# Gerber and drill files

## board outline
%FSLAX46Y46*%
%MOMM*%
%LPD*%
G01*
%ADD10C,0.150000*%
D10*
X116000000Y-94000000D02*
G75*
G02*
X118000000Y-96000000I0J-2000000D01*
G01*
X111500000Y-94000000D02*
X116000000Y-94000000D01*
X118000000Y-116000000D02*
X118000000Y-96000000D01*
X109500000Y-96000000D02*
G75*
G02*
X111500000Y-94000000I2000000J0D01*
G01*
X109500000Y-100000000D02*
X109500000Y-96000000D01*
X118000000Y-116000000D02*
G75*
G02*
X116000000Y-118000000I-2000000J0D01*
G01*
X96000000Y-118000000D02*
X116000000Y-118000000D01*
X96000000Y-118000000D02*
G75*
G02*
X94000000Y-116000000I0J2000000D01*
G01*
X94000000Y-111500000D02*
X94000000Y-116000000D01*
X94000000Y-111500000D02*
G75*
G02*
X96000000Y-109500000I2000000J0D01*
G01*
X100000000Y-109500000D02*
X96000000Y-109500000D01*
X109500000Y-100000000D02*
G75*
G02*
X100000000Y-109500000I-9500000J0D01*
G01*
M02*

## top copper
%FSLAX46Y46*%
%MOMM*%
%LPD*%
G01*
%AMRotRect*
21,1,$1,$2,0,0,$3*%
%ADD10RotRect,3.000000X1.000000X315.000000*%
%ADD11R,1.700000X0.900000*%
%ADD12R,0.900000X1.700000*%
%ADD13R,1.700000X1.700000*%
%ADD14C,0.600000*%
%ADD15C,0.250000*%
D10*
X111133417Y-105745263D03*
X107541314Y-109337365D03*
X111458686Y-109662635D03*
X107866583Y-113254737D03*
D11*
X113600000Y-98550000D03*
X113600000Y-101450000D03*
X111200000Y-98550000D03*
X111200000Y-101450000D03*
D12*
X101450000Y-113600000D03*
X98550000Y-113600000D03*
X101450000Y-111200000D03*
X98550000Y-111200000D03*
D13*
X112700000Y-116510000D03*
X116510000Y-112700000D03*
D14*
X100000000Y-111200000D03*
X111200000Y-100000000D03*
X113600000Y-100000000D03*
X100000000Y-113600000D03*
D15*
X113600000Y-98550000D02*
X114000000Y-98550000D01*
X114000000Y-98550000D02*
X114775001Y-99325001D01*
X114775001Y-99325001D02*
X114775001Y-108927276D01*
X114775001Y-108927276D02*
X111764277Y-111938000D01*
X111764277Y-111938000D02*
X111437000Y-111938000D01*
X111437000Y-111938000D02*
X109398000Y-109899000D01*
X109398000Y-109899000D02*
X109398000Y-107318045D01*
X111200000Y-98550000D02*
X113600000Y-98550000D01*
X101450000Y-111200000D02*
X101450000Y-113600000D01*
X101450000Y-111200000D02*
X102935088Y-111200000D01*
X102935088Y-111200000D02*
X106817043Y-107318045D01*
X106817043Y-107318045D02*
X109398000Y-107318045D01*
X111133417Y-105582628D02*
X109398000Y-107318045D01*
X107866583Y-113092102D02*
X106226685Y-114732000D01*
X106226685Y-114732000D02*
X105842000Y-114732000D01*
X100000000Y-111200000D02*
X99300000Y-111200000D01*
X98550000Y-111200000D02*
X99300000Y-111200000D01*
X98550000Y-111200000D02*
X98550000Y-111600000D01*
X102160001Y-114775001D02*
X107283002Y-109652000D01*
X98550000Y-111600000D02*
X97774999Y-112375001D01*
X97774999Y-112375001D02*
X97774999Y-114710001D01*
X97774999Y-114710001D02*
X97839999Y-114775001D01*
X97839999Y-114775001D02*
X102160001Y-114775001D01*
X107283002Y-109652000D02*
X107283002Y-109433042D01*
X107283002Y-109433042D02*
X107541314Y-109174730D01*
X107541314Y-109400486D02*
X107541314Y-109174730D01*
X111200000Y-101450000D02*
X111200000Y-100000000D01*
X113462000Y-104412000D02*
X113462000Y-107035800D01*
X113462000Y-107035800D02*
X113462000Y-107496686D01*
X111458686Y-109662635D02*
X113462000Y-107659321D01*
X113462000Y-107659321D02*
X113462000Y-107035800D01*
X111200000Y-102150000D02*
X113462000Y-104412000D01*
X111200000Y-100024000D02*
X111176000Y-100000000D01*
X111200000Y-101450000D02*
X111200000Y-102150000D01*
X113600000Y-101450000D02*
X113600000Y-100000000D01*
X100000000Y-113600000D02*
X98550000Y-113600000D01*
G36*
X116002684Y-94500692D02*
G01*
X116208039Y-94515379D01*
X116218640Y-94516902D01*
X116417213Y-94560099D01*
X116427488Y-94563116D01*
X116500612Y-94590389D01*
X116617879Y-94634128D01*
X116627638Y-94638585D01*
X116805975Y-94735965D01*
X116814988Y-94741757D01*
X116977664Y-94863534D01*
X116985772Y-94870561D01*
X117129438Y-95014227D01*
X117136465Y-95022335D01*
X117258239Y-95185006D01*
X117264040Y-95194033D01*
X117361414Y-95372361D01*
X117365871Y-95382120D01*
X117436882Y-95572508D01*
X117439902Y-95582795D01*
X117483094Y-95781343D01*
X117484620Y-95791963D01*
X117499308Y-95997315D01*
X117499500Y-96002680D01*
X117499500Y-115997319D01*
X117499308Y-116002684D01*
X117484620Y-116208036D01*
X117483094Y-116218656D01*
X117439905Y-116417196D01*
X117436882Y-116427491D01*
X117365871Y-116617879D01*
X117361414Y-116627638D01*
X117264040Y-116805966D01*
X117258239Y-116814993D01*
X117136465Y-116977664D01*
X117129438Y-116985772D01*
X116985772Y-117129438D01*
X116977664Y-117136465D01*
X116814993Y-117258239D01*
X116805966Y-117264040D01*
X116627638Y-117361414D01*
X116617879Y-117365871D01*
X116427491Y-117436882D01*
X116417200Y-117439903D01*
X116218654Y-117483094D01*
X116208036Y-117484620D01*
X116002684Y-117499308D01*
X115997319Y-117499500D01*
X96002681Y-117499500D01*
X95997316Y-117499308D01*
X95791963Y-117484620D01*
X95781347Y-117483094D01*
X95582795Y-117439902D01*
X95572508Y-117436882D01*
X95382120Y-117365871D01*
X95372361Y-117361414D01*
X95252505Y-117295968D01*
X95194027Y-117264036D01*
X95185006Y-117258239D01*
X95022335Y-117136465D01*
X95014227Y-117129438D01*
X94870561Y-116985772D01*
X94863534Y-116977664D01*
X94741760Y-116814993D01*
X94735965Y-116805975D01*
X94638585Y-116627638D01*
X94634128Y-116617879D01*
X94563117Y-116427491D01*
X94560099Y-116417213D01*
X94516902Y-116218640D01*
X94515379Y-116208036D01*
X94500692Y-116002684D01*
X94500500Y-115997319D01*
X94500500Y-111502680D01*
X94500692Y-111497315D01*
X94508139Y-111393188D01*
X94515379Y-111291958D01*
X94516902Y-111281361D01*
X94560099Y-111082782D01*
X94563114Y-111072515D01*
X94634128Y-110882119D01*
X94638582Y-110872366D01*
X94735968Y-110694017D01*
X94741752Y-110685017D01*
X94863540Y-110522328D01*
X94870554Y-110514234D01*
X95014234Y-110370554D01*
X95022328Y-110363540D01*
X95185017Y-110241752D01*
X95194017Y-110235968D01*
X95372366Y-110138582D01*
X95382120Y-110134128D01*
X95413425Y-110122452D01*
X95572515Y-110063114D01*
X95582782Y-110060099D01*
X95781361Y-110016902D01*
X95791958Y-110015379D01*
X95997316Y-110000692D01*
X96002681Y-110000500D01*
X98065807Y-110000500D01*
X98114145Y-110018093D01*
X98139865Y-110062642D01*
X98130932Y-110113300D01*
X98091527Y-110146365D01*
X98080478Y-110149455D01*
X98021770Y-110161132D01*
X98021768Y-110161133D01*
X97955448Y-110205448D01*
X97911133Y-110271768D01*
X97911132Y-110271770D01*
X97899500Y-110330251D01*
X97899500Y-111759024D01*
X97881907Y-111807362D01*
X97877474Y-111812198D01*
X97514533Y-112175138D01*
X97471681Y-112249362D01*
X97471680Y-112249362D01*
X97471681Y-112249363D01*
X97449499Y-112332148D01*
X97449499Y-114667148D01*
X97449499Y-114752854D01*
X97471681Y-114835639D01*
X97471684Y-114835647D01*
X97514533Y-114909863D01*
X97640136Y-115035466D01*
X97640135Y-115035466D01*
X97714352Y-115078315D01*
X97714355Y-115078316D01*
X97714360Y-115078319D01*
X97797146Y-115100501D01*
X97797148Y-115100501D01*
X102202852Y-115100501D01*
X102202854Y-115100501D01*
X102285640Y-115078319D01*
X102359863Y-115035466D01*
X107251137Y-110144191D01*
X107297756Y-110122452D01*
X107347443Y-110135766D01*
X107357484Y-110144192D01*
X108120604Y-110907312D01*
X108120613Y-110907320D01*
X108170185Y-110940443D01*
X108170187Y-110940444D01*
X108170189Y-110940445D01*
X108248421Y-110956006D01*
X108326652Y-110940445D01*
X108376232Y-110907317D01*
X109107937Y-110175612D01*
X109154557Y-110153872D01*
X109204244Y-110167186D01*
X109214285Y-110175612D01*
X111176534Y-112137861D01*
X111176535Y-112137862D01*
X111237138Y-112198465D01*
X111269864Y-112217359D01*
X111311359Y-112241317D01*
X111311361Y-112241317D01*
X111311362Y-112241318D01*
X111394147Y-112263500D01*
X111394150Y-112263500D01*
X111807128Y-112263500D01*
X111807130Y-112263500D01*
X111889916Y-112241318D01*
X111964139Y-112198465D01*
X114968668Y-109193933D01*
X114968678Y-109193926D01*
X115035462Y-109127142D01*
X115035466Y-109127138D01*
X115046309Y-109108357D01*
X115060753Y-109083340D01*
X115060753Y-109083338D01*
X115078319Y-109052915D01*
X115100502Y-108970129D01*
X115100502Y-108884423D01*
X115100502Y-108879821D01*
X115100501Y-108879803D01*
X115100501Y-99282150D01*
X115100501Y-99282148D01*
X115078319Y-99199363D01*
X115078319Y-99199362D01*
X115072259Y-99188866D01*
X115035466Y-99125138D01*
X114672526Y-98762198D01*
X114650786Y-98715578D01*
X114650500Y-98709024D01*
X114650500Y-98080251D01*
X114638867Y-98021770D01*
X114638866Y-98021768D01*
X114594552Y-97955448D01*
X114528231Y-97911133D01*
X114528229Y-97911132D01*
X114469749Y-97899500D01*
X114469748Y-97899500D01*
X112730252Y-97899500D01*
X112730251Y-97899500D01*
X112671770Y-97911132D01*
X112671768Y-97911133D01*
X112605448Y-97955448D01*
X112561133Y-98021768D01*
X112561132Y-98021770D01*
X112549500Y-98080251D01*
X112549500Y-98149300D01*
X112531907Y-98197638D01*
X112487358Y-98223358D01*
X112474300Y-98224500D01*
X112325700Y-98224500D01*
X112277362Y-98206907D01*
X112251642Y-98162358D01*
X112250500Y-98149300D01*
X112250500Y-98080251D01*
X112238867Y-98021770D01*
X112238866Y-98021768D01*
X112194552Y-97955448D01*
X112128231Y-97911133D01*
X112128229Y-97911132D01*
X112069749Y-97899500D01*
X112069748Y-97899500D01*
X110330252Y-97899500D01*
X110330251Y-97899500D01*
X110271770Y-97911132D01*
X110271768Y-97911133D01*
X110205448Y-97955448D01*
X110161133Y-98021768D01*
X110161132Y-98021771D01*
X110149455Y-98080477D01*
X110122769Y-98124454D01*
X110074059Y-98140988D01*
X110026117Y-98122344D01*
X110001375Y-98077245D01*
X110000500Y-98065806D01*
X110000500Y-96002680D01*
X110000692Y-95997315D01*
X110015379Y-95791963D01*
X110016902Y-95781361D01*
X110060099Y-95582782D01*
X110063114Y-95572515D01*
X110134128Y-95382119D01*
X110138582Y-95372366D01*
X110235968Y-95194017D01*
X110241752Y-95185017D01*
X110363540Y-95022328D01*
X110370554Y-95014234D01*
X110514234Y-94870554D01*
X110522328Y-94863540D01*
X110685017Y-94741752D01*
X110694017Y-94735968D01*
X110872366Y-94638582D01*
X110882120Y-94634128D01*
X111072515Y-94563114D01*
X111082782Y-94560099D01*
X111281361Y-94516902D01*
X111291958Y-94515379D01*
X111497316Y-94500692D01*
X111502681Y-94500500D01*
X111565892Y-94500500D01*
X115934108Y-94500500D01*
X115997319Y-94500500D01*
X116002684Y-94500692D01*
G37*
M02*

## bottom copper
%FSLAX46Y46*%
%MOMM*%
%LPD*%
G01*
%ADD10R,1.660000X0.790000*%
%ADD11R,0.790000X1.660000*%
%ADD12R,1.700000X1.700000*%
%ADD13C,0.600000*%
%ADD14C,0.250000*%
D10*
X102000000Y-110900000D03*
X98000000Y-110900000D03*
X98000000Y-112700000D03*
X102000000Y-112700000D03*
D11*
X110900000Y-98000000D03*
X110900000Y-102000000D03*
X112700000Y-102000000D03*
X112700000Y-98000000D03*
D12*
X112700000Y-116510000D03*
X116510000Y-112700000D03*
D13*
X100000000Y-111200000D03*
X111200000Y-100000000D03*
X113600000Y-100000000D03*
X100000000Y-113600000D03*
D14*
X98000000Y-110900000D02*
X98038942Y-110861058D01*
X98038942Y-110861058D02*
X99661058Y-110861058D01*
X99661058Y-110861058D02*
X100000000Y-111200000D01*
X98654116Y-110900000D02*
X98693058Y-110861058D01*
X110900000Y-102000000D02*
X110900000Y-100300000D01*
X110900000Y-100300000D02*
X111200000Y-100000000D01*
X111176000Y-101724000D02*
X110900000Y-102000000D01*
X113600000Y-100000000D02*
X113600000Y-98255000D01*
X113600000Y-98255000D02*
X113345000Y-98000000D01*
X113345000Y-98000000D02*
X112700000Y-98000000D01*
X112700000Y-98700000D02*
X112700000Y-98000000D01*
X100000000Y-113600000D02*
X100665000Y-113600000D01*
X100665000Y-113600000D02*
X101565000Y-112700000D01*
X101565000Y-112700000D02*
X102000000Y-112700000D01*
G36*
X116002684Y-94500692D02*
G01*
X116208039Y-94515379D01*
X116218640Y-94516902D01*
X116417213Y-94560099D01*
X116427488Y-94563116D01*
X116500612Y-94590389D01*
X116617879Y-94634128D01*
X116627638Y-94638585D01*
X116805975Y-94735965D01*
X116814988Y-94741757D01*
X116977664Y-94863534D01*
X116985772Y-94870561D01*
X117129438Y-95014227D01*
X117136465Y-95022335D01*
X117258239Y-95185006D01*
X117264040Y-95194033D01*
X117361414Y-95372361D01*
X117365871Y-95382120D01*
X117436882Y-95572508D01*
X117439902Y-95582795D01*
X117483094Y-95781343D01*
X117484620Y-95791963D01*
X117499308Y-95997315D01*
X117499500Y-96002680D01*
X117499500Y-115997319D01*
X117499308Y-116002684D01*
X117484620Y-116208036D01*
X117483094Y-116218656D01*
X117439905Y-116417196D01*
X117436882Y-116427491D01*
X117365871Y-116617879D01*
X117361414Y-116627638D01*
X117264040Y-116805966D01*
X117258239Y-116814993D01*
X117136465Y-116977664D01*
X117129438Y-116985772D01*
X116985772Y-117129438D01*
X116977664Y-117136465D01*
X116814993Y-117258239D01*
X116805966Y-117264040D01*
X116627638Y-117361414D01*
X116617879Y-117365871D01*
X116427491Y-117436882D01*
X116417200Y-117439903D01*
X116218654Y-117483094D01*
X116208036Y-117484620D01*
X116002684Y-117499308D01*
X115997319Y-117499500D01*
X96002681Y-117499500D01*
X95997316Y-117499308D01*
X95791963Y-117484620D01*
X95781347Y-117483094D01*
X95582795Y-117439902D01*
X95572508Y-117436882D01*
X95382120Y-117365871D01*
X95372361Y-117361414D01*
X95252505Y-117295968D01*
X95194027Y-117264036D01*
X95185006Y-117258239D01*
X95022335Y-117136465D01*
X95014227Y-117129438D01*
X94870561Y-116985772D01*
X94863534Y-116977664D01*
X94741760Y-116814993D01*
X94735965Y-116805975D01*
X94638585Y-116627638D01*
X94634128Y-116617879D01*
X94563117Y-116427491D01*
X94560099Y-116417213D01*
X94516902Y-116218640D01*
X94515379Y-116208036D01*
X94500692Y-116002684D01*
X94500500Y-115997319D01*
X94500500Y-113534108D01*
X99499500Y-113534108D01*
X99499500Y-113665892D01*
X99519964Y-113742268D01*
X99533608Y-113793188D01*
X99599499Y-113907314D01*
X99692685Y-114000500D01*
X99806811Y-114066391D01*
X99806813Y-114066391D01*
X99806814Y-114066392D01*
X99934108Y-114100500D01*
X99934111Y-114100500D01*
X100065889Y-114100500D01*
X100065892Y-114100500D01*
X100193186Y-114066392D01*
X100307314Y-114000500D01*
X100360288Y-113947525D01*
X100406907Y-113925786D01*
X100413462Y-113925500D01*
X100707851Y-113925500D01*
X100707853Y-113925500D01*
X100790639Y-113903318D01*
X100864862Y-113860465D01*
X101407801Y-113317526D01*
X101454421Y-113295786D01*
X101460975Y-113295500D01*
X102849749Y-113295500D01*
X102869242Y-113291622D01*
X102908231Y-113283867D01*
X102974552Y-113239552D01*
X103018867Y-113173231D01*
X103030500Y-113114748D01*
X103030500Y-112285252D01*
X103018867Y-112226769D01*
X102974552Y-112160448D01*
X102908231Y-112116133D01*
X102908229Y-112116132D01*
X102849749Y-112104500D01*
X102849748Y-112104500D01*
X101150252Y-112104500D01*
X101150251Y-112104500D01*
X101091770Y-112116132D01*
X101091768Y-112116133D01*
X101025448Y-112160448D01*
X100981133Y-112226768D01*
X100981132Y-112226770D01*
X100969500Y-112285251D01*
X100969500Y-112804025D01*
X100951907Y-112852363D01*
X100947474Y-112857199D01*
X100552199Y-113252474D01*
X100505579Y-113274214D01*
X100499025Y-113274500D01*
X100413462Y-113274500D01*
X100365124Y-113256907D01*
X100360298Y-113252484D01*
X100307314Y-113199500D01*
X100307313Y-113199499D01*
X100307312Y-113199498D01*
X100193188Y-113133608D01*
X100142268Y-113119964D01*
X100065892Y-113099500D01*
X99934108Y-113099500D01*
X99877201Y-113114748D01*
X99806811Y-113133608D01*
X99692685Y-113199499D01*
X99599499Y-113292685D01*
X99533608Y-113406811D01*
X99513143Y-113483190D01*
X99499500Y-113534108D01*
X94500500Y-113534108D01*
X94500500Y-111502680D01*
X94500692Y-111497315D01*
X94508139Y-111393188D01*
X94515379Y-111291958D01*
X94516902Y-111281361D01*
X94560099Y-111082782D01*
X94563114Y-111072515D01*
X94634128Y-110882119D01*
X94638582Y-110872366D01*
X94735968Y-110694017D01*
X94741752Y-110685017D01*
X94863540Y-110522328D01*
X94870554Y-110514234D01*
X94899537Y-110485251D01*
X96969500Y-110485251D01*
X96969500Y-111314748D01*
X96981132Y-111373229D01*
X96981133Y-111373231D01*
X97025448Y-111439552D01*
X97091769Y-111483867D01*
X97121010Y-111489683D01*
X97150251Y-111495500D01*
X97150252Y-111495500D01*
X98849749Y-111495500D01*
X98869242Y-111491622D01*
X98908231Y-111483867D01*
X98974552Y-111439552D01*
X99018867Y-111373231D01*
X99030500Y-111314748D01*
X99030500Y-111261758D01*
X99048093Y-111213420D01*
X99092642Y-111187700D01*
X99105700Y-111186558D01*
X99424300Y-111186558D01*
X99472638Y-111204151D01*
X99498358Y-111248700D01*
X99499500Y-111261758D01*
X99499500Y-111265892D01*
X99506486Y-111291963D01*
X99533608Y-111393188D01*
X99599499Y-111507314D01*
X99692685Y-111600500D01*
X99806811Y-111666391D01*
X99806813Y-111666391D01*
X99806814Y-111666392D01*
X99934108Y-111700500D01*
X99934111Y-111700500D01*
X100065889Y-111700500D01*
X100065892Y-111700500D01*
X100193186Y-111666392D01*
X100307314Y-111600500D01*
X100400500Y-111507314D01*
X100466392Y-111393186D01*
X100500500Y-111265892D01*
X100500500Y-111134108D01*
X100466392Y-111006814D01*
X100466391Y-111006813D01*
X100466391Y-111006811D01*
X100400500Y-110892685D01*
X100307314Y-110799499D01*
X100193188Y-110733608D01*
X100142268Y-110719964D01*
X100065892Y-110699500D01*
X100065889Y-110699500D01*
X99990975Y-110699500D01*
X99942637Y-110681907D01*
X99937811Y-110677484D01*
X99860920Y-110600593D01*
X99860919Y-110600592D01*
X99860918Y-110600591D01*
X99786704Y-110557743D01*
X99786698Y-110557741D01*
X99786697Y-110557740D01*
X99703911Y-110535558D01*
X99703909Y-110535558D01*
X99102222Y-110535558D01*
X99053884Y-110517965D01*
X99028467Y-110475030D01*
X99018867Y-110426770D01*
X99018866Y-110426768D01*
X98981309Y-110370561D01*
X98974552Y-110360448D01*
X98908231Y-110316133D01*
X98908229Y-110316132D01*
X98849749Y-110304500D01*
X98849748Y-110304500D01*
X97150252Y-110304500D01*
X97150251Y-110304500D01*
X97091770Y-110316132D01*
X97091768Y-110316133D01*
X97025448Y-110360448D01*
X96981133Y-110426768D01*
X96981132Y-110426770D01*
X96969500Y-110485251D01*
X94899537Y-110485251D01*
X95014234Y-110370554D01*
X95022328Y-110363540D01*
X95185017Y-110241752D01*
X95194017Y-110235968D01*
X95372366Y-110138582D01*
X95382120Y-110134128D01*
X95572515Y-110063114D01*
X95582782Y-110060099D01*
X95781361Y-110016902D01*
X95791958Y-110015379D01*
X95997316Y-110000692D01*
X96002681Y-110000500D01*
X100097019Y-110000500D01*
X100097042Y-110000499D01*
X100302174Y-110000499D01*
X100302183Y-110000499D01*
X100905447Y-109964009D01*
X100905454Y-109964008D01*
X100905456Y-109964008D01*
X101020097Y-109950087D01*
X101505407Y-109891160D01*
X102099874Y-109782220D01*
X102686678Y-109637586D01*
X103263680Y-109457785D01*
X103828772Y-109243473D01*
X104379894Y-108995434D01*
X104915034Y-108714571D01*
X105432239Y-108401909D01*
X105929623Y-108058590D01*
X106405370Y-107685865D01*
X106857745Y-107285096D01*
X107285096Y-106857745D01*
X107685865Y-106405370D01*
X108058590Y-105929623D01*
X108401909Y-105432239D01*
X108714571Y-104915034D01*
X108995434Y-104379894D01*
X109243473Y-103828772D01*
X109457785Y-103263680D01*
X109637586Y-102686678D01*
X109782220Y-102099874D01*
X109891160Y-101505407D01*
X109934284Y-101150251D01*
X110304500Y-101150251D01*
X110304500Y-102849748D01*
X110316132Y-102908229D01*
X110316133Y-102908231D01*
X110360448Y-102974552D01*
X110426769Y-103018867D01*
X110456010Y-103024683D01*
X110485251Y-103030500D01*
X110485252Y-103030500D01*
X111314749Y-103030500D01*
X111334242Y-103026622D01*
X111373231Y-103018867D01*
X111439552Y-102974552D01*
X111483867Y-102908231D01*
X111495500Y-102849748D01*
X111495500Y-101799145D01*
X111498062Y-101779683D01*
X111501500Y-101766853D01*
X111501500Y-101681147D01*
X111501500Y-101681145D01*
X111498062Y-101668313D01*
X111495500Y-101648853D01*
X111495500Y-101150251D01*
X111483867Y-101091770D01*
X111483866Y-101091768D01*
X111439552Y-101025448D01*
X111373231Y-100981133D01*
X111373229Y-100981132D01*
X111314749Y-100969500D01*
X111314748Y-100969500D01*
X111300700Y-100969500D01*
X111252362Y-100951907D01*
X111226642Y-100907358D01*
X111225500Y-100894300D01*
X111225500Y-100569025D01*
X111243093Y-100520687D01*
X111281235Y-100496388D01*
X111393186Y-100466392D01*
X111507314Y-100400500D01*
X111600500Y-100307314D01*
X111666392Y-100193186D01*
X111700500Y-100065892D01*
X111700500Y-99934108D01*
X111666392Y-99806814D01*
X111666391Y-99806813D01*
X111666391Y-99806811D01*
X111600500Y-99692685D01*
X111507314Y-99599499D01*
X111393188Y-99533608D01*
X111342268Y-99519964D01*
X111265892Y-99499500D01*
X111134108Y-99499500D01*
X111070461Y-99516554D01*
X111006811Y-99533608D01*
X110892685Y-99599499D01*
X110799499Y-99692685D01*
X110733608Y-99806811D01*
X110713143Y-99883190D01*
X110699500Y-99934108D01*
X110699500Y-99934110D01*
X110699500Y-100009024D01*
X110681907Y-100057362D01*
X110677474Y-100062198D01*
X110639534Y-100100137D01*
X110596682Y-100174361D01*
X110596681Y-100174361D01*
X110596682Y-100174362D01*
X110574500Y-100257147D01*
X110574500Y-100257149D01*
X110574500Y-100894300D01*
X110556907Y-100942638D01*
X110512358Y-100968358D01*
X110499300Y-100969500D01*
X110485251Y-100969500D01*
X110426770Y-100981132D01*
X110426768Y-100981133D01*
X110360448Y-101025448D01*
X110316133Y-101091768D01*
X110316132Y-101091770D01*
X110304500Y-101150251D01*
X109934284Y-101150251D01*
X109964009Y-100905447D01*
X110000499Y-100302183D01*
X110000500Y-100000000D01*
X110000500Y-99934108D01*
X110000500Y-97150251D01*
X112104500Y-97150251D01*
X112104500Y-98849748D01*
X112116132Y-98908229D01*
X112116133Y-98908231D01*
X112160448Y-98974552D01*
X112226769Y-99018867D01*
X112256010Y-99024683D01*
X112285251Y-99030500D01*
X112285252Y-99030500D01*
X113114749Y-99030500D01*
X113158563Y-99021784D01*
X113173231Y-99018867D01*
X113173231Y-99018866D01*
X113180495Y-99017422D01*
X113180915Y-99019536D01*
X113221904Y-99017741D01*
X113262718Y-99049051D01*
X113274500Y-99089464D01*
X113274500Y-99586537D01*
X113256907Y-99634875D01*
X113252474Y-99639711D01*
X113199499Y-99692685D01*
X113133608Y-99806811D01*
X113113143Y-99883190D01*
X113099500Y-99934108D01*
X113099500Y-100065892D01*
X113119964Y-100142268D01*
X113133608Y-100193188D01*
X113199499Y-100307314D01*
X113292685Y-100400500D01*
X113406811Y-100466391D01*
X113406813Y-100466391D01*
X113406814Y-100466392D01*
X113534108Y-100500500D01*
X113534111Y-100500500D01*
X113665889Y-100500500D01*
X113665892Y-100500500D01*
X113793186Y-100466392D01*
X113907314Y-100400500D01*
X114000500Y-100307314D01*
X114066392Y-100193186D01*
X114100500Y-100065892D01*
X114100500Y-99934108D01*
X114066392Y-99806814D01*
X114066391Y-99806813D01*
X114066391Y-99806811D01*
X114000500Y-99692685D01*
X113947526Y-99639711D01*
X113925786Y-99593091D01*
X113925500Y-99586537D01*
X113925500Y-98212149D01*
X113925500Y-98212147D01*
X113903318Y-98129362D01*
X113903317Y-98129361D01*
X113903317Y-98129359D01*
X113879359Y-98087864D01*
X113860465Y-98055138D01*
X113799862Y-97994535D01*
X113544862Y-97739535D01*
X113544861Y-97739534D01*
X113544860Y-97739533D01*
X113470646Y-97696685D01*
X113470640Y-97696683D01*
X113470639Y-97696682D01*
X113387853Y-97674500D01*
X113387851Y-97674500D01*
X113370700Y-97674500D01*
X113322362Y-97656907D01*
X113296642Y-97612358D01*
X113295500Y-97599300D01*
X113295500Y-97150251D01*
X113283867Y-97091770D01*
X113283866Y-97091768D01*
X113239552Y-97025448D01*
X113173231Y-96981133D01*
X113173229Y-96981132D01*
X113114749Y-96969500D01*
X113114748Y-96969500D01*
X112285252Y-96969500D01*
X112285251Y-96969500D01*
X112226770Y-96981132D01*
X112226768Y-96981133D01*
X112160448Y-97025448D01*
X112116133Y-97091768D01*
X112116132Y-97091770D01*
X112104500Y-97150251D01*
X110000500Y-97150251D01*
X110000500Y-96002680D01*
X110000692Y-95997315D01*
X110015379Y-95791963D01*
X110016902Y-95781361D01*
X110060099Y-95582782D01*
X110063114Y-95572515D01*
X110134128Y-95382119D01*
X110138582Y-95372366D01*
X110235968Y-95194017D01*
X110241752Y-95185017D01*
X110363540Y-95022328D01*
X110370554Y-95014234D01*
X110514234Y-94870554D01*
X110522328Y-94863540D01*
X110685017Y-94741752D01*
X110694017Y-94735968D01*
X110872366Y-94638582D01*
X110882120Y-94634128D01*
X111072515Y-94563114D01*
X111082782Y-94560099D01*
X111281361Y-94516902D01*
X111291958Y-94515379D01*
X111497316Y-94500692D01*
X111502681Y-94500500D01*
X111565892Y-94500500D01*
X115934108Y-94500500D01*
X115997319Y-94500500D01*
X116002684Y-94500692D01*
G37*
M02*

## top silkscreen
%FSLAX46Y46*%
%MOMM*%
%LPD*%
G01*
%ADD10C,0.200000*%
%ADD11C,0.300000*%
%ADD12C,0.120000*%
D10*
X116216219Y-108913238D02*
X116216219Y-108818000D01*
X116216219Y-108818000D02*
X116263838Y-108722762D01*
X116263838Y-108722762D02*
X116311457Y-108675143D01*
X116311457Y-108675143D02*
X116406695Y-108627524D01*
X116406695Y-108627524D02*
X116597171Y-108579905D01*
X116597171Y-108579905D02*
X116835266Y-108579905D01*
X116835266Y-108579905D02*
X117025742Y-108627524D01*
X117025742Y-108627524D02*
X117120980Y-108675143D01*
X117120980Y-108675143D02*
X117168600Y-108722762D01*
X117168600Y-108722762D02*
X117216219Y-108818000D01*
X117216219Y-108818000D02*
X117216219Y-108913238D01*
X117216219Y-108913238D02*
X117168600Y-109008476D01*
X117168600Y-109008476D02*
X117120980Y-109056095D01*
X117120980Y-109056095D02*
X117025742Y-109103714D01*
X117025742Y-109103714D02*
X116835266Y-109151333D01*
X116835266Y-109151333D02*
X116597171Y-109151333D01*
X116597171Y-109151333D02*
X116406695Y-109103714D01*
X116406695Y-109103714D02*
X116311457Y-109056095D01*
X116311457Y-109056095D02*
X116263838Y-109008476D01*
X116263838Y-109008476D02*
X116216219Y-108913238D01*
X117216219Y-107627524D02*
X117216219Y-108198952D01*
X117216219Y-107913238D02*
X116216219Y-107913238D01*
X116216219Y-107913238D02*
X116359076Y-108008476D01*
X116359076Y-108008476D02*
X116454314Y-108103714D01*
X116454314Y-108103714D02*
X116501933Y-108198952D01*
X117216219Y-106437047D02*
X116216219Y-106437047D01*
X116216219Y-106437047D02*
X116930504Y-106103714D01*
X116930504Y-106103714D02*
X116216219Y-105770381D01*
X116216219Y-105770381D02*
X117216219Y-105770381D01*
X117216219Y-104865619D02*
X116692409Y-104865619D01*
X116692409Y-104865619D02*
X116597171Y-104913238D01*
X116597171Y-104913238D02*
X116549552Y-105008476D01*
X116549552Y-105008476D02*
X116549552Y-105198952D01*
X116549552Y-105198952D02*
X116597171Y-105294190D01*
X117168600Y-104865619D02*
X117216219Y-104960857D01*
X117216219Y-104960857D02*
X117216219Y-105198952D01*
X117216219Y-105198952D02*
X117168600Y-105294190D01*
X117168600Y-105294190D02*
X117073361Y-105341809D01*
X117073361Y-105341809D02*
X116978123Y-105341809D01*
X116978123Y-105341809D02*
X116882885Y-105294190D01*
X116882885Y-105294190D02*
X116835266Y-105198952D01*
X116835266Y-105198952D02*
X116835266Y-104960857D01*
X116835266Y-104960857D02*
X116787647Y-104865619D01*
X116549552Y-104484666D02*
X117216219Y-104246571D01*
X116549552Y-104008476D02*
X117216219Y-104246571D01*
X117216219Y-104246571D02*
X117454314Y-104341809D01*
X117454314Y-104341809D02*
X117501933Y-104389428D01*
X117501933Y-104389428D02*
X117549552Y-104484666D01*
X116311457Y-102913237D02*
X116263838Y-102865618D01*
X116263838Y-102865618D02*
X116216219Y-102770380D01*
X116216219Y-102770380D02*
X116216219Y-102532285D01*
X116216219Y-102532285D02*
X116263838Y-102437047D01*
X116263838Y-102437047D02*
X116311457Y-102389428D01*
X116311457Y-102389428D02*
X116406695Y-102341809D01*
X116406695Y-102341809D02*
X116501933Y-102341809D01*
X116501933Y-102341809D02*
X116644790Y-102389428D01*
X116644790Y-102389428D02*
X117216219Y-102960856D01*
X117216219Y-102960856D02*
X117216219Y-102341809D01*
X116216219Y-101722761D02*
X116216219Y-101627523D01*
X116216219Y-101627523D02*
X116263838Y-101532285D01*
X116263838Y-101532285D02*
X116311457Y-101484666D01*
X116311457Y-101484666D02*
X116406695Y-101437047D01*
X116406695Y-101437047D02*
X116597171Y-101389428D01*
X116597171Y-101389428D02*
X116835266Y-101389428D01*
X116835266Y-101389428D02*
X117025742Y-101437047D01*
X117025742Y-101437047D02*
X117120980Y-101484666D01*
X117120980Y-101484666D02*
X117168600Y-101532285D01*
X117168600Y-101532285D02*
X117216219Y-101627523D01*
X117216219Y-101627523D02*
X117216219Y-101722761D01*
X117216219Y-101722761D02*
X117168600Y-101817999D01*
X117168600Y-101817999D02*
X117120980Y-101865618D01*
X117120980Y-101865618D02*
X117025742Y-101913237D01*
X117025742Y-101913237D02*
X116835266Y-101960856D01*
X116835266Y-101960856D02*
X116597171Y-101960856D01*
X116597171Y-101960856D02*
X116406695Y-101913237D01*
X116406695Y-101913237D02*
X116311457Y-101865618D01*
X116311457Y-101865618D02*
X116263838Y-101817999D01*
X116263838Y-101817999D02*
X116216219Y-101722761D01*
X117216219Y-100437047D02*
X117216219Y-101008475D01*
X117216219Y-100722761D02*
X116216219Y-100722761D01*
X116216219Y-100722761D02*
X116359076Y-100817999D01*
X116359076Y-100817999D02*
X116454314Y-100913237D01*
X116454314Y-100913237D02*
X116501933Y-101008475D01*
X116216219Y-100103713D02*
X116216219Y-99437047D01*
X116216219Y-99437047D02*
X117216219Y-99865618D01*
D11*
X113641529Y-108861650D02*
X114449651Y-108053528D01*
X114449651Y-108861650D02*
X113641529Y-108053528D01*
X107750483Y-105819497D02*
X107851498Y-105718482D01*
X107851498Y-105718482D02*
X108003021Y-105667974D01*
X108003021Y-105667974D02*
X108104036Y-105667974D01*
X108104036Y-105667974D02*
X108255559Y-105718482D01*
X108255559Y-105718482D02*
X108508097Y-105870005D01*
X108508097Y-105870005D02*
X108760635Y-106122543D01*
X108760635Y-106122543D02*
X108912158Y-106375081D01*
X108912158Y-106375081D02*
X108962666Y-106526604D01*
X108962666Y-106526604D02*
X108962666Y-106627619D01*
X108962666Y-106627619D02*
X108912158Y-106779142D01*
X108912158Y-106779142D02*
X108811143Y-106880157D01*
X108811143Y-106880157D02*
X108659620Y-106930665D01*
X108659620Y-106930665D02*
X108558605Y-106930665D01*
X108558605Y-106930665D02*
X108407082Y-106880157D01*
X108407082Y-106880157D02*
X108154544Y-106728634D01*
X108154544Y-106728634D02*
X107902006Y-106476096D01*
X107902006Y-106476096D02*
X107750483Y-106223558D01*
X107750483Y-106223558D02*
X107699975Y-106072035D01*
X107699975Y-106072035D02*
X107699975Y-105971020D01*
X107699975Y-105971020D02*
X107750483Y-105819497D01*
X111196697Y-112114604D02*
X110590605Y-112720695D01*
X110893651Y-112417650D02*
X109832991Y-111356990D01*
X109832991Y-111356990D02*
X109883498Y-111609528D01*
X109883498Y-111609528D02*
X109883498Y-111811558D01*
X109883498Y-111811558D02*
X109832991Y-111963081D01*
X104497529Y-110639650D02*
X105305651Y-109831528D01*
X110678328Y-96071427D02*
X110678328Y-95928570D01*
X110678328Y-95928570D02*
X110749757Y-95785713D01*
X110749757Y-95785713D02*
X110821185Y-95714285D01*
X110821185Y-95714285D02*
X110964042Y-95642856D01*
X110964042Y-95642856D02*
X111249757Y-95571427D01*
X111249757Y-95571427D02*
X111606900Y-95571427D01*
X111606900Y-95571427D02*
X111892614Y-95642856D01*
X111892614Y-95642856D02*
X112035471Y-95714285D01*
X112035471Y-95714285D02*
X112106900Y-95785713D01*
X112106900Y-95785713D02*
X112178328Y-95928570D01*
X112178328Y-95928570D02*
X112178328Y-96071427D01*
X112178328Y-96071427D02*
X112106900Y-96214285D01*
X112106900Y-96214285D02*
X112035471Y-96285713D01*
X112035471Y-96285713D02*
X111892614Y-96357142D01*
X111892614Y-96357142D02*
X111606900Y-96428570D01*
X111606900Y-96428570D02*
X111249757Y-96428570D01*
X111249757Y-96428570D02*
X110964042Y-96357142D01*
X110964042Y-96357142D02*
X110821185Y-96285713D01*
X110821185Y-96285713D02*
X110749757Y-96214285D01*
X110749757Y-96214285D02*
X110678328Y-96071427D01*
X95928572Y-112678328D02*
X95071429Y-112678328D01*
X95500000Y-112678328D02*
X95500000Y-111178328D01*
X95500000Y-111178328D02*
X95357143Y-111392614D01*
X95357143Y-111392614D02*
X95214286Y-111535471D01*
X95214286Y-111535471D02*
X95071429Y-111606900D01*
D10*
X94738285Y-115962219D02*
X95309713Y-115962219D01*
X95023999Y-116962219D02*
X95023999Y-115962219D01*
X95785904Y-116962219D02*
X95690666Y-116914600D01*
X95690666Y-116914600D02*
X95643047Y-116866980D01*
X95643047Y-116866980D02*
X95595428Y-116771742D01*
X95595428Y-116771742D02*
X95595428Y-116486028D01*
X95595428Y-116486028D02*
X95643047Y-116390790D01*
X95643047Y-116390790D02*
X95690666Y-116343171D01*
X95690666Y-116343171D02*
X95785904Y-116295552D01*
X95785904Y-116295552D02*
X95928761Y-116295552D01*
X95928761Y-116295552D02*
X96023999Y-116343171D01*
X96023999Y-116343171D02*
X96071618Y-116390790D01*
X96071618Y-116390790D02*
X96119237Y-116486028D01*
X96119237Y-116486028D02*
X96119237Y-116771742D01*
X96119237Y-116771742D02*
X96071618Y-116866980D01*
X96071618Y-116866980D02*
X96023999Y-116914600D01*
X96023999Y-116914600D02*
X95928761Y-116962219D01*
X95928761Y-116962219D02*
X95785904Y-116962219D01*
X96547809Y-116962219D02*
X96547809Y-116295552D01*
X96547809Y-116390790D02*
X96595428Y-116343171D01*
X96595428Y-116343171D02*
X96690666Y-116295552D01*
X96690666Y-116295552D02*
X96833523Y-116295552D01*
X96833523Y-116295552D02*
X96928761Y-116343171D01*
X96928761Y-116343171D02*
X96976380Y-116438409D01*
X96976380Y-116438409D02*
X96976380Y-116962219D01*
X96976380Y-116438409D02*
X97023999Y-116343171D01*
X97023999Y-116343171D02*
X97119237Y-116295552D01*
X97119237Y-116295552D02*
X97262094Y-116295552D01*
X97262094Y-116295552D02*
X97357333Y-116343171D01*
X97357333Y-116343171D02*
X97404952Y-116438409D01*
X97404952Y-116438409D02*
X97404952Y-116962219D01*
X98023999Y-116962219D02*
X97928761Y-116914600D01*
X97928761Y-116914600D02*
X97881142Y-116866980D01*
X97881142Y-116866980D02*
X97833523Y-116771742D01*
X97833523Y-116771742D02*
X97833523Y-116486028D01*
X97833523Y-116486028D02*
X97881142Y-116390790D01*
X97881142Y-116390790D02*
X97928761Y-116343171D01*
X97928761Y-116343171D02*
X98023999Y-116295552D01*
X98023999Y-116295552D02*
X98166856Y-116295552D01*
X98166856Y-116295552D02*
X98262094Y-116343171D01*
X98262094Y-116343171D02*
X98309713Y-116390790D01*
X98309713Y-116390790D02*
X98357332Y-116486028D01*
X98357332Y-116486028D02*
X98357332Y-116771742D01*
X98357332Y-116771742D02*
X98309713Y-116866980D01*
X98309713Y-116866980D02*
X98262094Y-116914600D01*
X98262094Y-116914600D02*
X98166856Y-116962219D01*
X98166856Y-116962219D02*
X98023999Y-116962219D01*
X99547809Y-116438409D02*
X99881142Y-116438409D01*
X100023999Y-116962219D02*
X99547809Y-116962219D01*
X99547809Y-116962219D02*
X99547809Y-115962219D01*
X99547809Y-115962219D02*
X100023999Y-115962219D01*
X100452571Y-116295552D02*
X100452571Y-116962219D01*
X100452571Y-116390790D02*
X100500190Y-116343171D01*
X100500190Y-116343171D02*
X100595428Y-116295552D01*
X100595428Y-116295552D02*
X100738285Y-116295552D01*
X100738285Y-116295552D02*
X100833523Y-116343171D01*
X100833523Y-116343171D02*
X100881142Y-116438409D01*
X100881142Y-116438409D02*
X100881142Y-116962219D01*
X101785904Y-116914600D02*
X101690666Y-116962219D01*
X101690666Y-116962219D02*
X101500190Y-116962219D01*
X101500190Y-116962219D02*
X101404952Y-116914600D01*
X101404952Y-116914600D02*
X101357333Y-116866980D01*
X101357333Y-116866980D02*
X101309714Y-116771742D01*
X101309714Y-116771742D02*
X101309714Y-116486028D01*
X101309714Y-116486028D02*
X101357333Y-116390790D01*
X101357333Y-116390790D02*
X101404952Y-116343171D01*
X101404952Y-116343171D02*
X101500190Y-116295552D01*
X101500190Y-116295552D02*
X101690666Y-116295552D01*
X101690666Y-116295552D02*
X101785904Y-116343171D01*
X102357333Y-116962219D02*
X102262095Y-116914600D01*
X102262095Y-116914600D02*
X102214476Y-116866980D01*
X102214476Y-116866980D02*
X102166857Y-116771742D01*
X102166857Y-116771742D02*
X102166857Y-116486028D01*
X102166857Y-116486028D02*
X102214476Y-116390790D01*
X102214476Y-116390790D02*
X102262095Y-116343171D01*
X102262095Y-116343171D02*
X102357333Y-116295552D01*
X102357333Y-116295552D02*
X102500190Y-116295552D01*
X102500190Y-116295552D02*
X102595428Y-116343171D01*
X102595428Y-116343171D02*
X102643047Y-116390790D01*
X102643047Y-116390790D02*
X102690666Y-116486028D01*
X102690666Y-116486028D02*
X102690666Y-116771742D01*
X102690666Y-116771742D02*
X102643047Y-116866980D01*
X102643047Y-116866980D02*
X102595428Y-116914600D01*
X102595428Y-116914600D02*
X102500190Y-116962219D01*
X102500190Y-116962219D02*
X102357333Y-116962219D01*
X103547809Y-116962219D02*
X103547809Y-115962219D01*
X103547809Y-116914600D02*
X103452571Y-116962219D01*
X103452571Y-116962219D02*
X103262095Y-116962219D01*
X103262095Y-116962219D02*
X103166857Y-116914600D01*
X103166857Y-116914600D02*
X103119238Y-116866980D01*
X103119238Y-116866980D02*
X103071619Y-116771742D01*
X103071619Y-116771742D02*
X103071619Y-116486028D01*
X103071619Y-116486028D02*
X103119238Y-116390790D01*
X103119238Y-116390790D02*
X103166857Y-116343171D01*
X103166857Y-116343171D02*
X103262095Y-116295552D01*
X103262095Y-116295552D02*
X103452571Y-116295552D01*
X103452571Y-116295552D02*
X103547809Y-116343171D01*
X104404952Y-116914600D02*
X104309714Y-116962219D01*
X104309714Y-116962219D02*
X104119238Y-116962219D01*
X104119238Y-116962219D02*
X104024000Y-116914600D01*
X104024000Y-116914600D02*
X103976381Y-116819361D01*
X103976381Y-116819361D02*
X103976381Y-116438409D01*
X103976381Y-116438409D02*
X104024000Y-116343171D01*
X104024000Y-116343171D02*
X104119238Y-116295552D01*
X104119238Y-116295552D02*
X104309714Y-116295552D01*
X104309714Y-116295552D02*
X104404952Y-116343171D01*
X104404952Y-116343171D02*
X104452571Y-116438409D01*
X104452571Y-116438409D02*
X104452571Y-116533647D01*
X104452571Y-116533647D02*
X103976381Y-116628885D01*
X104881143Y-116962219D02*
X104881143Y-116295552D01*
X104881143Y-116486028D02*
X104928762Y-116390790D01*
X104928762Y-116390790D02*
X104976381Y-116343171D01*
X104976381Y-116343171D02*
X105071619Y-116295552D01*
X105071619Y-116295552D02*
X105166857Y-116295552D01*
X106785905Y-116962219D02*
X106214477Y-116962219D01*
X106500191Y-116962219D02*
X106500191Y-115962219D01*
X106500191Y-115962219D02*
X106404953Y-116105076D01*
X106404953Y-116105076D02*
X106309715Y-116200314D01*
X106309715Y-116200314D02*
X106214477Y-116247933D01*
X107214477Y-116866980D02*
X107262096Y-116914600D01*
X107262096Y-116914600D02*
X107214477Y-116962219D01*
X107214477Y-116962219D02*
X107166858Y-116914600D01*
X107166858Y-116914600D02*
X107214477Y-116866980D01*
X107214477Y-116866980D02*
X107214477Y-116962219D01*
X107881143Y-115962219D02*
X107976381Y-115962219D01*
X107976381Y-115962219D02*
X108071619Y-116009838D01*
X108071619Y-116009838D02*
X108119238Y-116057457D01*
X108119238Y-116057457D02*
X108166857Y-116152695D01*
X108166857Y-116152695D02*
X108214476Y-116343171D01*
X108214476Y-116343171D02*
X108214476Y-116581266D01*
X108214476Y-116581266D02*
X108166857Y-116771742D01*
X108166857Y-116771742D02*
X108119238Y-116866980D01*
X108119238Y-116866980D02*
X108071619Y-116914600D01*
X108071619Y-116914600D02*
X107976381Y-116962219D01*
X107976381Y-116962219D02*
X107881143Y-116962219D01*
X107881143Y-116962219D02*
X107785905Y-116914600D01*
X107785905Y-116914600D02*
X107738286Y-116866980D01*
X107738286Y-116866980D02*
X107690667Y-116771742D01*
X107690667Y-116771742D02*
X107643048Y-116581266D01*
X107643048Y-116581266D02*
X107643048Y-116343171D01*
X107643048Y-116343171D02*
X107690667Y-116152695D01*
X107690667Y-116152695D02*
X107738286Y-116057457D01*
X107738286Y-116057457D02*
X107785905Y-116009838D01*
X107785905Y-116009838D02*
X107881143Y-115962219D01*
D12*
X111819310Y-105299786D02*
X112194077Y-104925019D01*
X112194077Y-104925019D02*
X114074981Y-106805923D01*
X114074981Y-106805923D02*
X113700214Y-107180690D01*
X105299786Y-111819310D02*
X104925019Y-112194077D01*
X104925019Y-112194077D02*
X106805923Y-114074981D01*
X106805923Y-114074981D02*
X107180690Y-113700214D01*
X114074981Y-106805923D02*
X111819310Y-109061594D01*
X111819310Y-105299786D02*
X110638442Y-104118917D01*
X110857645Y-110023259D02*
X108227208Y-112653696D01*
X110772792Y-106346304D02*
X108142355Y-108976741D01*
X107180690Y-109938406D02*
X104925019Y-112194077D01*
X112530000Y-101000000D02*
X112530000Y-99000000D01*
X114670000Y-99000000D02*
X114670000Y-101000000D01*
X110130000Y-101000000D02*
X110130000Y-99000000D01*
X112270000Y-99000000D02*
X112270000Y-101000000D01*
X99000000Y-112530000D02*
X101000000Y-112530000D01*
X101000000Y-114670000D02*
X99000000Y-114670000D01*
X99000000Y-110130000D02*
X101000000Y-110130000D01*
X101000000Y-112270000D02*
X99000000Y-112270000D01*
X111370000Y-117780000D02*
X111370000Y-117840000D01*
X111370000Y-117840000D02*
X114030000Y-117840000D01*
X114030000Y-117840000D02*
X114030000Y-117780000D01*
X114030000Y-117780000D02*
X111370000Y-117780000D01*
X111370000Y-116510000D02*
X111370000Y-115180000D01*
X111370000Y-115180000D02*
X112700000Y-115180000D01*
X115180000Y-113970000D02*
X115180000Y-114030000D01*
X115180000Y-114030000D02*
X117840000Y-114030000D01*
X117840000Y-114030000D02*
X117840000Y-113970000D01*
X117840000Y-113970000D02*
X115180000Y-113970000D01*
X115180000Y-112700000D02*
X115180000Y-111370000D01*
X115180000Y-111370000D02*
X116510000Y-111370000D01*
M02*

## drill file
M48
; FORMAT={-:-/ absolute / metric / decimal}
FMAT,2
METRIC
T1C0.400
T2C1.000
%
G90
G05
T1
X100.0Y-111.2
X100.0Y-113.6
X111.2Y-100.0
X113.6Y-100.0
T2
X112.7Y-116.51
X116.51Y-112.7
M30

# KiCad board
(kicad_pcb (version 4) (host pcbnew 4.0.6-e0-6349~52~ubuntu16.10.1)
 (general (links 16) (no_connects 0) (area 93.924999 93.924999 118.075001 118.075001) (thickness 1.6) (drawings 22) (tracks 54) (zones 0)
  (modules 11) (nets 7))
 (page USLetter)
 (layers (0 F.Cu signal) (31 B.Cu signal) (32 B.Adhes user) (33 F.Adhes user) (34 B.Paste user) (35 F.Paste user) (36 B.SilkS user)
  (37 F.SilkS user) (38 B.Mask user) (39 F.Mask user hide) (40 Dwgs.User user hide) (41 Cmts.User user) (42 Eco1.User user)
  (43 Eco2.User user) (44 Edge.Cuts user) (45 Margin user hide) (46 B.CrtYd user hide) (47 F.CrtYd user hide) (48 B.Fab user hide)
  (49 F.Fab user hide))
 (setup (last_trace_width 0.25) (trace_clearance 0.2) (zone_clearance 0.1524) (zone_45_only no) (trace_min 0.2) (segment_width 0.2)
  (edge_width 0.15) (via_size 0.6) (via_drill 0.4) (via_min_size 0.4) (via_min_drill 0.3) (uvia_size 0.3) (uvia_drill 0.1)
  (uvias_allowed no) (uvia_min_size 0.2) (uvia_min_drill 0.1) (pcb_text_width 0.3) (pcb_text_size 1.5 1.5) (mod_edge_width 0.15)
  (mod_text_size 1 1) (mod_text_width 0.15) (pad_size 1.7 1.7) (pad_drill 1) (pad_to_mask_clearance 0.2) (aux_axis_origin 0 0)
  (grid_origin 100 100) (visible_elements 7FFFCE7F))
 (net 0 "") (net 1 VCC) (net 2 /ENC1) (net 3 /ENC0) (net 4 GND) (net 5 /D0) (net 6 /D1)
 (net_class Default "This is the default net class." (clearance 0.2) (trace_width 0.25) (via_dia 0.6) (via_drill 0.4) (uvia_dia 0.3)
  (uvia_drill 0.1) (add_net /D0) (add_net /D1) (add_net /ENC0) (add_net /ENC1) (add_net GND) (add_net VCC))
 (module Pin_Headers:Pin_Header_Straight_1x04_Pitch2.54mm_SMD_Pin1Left (layer F.Cu) (at 109.5 109.5 315)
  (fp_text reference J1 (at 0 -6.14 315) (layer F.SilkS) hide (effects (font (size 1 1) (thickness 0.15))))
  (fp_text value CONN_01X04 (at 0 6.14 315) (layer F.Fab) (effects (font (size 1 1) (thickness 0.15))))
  (fp_line (start -1.33 -4.61) (end -1.33 -5.14) (layer F.SilkS) (width 0.12))
  (fp_line (start -1.33 -5.14) (end 1.33 -5.14) (layer F.SilkS) (width 0.12))
  (fp_line (start 1.33 -5.14) (end 1.33 -4.61) (layer F.SilkS) (width 0.12))
  (fp_line (start -1.33 4.61) (end -1.33 5.14) (layer F.SilkS) (width 0.12))
  (fp_line (start -1.33 5.14) (end 1.33 5.14) (layer F.SilkS) (width 0.12))
  (fp_line (start 1.33 5.14) (end 1.33 4.61) (layer F.SilkS) (width 0.12))
  (fp_line (start 1.33 -5.14) (end 1.33 -1.95) (layer F.SilkS) (width 0.12))
  (fp_line (start -1.33 -4.61) (end -3 -4.61) (layer F.SilkS) (width 0.12))
  (fp_line (start 1.33 -0.59) (end 1.33 3.13) (layer F.SilkS) (width 0.12))
  (fp_line (start -1.33 -3.13) (end -1.33 0.59) (layer F.SilkS) (width 0.12))
  (fp_line (start -1.33 1.95) (end -1.33 5.14) (layer F.SilkS) (width 0.12))
  (pad 1 smd rect (at -1.5 -3.81 315) (size 3 1) (layers F.Cu F.Paste F.Mask) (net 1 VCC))
  (pad 3 smd rect (at -1.5 1.27 315) (size 3 1) (layers F.Cu F.Paste F.Mask) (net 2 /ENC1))
  (pad 2 smd rect (at 1.5 -1.27 315) (size 3 1) (layers F.Cu F.Paste F.Mask) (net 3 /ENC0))
  (pad 4 smd rect (at 1.5 3.81 315) (size 3 1) (layers F.Cu F.Paste F.Mask) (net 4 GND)))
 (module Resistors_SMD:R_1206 (layer F.Cu) (at 113.6 100 270)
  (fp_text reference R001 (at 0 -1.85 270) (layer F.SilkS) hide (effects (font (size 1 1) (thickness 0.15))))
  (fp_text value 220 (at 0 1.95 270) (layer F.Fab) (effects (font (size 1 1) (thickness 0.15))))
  (fp_line (start 1 1.07) (end -1 1.07) (layer F.SilkS) (width 0.12))
  (fp_line (start -1 -1.07) (end 1 -1.07) (layer F.SilkS) (width 0.12))
  (pad 1 smd rect (at -1.45 0 270) (size 0.9 1.7) (layers F.Cu F.Paste F.Mask) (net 1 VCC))
  (pad 2 smd rect (at 1.45 0 270) (size 0.9 1.7) (layers F.Cu F.Paste F.Mask) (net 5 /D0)))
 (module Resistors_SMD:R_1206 (layer F.Cu) (at 111.2 100 270)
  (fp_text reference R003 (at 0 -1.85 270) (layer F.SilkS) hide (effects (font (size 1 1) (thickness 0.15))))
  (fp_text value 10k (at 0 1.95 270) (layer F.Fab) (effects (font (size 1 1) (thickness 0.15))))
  (fp_line (start 1 1.07) (end -1 1.07) (layer F.SilkS) (width 0.12))
  (fp_line (start -1 -1.07) (end 1 -1.07) (layer F.SilkS) (width 0.12))
  (pad 1 smd rect (at -1.45 0 270) (size 0.9 1.7) (layers F.Cu F.Paste F.Mask) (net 1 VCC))
  (pad 2 smd rect (at 1.45 0 270) (size 0.9 1.7) (layers F.Cu F.Paste F.Mask) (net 3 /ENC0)))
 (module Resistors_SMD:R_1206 (layer F.Cu) (at 100 113.6 180)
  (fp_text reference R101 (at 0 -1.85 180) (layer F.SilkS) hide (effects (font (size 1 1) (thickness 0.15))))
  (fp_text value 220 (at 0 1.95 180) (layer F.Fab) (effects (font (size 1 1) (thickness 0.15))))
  (fp_line (start 1 1.07) (end -1 1.07) (layer F.SilkS) (width 0.12))
  (fp_line (start -1 -1.07) (end 1 -1.07) (layer F.SilkS) (width 0.12))
  (pad 1 smd rect (at -1.45 0 180) (size 0.9 1.7) (layers F.Cu F.Paste F.Mask) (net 1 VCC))
  (pad 2 smd rect (at 1.45 0 180) (size 0.9 1.7) (layers F.Cu F.Paste F.Mask) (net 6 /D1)))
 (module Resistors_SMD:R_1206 (layer F.Cu) (at 100 111.2 180)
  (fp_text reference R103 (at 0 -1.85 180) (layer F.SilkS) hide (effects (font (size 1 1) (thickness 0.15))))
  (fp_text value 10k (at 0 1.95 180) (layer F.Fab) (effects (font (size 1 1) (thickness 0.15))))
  (fp_line (start 1 1.07) (end -1 1.07) (layer F.SilkS) (width 0.12))
  (fp_line (start -1 -1.07) (end 1 -1.07) (layer F.SilkS) (width 0.12))
  (pad 1 smd rect (at -1.45 0 180) (size 0.9 1.7) (layers F.Cu F.Paste F.Mask) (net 1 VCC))
  (pad 2 smd rect (at 1.45 0 180) (size 0.9 1.7) (layers F.Cu F.Paste F.Mask) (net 2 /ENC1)))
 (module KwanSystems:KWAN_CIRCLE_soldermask (layer B.Cu) (at 113.716 107.874 180)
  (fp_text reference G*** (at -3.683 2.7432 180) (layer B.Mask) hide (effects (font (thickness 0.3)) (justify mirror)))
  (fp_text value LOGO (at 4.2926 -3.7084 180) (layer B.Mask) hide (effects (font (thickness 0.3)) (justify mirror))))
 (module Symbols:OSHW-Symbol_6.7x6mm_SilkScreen (layer B.Cu) (at 107.62 114.478 180)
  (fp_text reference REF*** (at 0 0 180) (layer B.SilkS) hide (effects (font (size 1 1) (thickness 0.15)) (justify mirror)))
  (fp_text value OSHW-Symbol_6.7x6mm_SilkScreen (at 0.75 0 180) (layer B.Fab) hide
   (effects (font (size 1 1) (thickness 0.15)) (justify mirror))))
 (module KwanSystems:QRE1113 (layer B.Cu) (at 100 111.8 180)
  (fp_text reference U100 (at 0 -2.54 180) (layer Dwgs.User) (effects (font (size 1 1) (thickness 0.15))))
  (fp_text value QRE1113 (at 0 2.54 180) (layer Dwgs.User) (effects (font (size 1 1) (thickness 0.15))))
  (pad 4 smd rect (at -2 0.9 180) (size 1.66 0.79) (layers B.Cu B.Paste B.Mask) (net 4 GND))
  (pad 3 smd rect (at 2 0.9 180) (size 1.66 0.79) (layers B.Cu B.Paste B.Mask) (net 2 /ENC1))
  (pad 2 smd rect (at 2 -0.9 180) (size 1.66 0.79) (layers B.Cu B.Paste B.Mask) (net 4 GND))
  (pad 1 smd rect (at -2 -0.9 180) (size 1.66 0.79) (layers B.Cu B.Paste B.Mask) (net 6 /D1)))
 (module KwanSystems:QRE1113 (layer B.Cu) (at 111.8 100 270)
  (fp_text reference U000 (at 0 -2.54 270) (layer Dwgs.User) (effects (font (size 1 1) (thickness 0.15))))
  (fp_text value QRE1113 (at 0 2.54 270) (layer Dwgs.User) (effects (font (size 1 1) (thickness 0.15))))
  (pad 4 smd rect (at -2 0.9 270) (size 1.66 0.79) (layers B.Cu B.Paste B.Mask) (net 4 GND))
  (pad 3 smd rect (at 2 0.9 270) (size 1.66 0.79) (layers B.Cu B.Paste B.Mask) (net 3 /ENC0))
  (pad 2 smd rect (at 2 -0.9 270) (size 1.66 0.79) (layers B.Cu B.Paste B.Mask) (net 4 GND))
  (pad 1 smd rect (at -2 -0.9 270) (size 1.66 0.79) (layers B.Cu B.Paste B.Mask) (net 5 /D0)))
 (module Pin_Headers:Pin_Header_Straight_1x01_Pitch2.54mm (layer F.Cu) (at 112.7 116.51)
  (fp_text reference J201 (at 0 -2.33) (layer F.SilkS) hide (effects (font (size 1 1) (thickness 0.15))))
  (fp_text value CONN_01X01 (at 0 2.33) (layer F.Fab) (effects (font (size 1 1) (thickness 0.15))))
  (fp_line (start -1.33 1.27) (end -1.33 1.33) (layer F.SilkS) (width 0.12))
  (fp_line (start -1.33 1.33) (end 1.33 1.33) (layer F.SilkS) (width 0.12))
  (fp_line (start 1.33 1.33) (end 1.33 1.27) (layer F.SilkS) (width 0.12))
  (fp_line (start 1.33 1.27) (end -1.33 1.27) (layer F.SilkS) (width 0.12))
  (fp_line (start -1.33 0) (end -1.33 -1.33) (layer F.SilkS) (width 0.12))
  (fp_line (start -1.33 -1.33) (end 0 -1.33) (layer F.SilkS) (width 0.12))
  (pad 1 thru_hole rect (at 0 0) (size 1.7 1.7) (drill 1) (layers *.Cu *.Mask) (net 4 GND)))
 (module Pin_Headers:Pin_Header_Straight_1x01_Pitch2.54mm (layer F.Cu) (at 116.51 112.7)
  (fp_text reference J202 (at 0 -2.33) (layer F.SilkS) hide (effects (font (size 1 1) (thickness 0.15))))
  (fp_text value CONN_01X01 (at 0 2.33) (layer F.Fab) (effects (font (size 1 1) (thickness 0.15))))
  (fp_line (start -1.33 1.27) (end -1.33 1.33) (layer F.SilkS) (width 0.12))
  (fp_line (start -1.33 1.33) (end 1.33 1.33) (layer F.SilkS) (width 0.12))
  (fp_line (start 1.33 1.33) (end 1.33 1.27) (layer F.SilkS) (width 0.12))
  (fp_line (start 1.33 1.27) (end -1.33 1.27) (layer F.SilkS) (width 0.12))
  (fp_line (start -1.33 0) (end -1.33 -1.33) (layer F.SilkS) (width 0.12))
  (fp_line (start -1.33 -1.33) (end 0 -1.33) (layer F.SilkS) (width 0.12))
  (pad 1 thru_hole rect (at 0 0) (size 1.7 1.7) (drill 1) (layers *.Cu *.Mask) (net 4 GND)))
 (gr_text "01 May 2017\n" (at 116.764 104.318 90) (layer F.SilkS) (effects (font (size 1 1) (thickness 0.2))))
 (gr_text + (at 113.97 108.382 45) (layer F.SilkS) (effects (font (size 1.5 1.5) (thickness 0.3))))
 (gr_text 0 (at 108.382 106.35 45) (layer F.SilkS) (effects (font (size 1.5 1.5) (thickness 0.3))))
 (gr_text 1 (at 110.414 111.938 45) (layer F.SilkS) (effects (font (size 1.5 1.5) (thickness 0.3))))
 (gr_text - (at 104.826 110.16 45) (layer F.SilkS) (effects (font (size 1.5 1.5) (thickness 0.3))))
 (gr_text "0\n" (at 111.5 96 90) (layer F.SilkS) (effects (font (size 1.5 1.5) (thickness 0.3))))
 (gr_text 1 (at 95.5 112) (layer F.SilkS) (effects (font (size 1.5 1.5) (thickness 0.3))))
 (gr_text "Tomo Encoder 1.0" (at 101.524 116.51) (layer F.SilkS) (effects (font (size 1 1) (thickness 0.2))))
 (gr_arc (start 116 96) (end 116 94) (angle 90) (layer Edge.Cuts) (width 0.15))
 (gr_line (start 111.5 94) (end 116 94) (layer Edge.Cuts) (width 0.15))
 (gr_line (start 118 116) (end 118 96) (layer Edge.Cuts) (width 0.15))
 (gr_arc (start 111.5 96) (end 109.5 96) (angle 90) (layer Edge.Cuts) (width 0.15))
 (gr_line (start 109.5 100) (end 109.5 96) (layer Edge.Cuts) (width 0.15))
 (gr_arc (start 116 116) (end 118 116) (angle 90) (layer Edge.Cuts) (width 0.15))
 (gr_line (start 96 118) (end 116 118) (layer Edge.Cuts) (width 0.15))
 (gr_arc (start 96 116) (end 96 118) (angle 90) (layer Edge.Cuts) (width 0.15))
 (gr_line (start 94 111.5) (end 94 116) (layer Edge.Cuts) (width 0.15))
 (gr_arc (start 96 111.5) (end 94 111.5) (angle 90) (layer Edge.Cuts) (width 0.15))
 (gr_line (start 100 109.5) (end 96 109.5) (layer Edge.Cuts) (width 0.15))
 (gr_arc (start 100 100) (end 109.5 100) (angle 90) (layer Edge.Cuts) (width 0.15))
 (segment (start 113.6 98.55) (end 114 98.55) (width 0.25) (layer F.Cu) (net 1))
 (segment (start 114 98.55) (end 114.775001 99.325001) (width 0.25) (layer F.Cu) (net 1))
 (segment (start 114.775001 99.325001) (end 114.775001 108.927276) (width 0.25) (layer F.Cu) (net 1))
 (segment (start 114.775001 108.927276) (end 111.764277 111.938) (width 0.25) (layer F.Cu) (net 1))
 (segment (start 111.764277 111.938) (end 111.437 111.938) (width 0.25) (layer F.Cu) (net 1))
 (segment (start 111.437 111.938) (end 109.398 109.899) (width 0.25) (layer F.Cu) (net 1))
 (segment (start 109.398 109.899) (end 109.398 107.318045) (width 0.25) (layer F.Cu) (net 1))
 (segment (start 111.2 98.55) (end 113.6 98.55) (width 0.25) (layer F.Cu) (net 1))
 (segment (start 101.45 111.2) (end 101.45 113.6) (width 0.25) (layer F.Cu) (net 1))
 (segment (start 101.45 111.2) (end 102.935088 111.2) (width 0.25) (layer F.Cu) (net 1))
 (segment (start 102.935088 111.2) (end 106.817043 107.318045) (width 0.25) (layer F.Cu) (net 1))
 (segment (start 106.817043 107.318045) (end 109.398 107.318045) (width 0.25) (layer F.Cu) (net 1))
 (segment (start 111.133417 105.582628) (end 109.398 107.318045) (width 0.25) (layer F.Cu) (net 1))
 (segment (start 107.866583 113.092102) (end 106.226685 114.732) (width 0.25) (layer F.Cu) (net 4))
 (segment (start 106.226685 114.732) (end 105.842 114.732) (width 0.25) (layer F.Cu) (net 4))
 (segment (start 100 111.2) (end 99.3 111.2) (width 0.25) (layer F.Cu) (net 2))
 (segment (start 98.55 111.2) (end 99.3 111.2) (width 0.25) (layer F.Cu) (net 2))
 (segment (start 98 110.9) (end 98.038942 110.861058) (width 0.25) (layer B.Cu) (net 2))
 (segment (start 98.038942 110.861058) (end 99.661058 110.861058) (width 0.25) (layer B.Cu) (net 2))
 (segment (start 99.661058 110.861058) (end 100 111.2) (width 0.25) (layer B.Cu) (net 2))
 (segment (start 98.55 111.2) (end 98.55 111.6) (width 0.25) (layer F.Cu) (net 2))
 (segment (start 102.160001 114.775001) (end 107.283002 109.652) (width 0.25) (layer F.Cu) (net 2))
 (segment (start 98.55 111.6) (end 97.774999 112.375001) (width 0.25) (layer F.Cu) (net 2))
 (segment (start 97.774999 112.375001) (end 97.774999 114.710001) (width 0.25) (layer F.Cu) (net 2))
 (segment (start 97.774999 114.710001) (end 97.839999 114.775001) (width 0.25) (layer F.Cu) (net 2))
 (segment (start 97.839999 114.775001) (end 102.160001 114.775001) (width 0.25) (layer F.Cu) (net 2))
 (segment (start 107.283002 109.652) (end 107.283002 109.433042) (width 0.25) (layer F.Cu) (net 2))
 (segment (start 107.283002 109.433042) (end 107.541314 109.17473) (width 0.25) (layer F.Cu) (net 2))
 (segment (start 107.541314 109.400486) (end 107.541314 109.17473) (width 0.25) (layer F.Cu) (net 2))
 (segment (start 98.654116 110.9) (end 98.693058 110.861058) (width 0.25) (layer B.Cu) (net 2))
 (via (at 100 111.2) (size 0.6) (drill 0.4) (layers F.Cu B.Cu) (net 2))
 (segment (start 110.9 102) (end 110.9 100.3) (width 0.25) (layer B.Cu) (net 3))
 (segment (start 110.9 100.3) (end 111.2 100) (width 0.25) (layer B.Cu) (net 3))
 (segment (start 111.2 101.45) (end 111.2 100) (width 0.25) (layer F.Cu) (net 3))
 (segment (start 113.462 104.412) (end 113.462 107.0358) (width 0.25) (layer F.Cu) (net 3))
 (segment (start 113.462 107.0358) (end 113.462 107.496686) (width 0.25) (layer F.Cu) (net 3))
 (segment (start 111.458686 109.662635) (end 113.462 107.659321) (width 0.25) (layer F.Cu) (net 3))
 (segment (start 113.462 107.659321) (end 113.462 107.0358) (width 0.25) (layer F.Cu) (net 3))
 (segment (start 111.2 102.15) (end 113.462 104.412) (width 0.25) (layer F.Cu) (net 3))
 (segment (start 111.176 101.724) (end 110.9 102) (width 0.25) (layer B.Cu) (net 3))
 (segment (start 111.2 100.024) (end 111.176 100) (width 0.25) (layer F.Cu) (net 3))
 (via (at 111.2 100) (size 0.6) (drill 0.4) (layers F.Cu B.Cu) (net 3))
 (segment (start 111.2 101.45) (end 111.2 102.15) (width 0.25) (layer F.Cu) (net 3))
 (segment (start 113.6 100) (end 113.6 98.255) (width 0.25) (layer B.Cu) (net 5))
 (segment (start 113.6 98.255) (end 113.345 98) (width 0.25) (layer B.Cu) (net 5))
 (segment (start 113.345 98) (end 112.7 98) (width 0.25) (layer B.Cu) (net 5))
 (segment (start 113.6 101.45) (end 113.6 100) (width 0.25) (layer F.Cu) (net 5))
 (segment (start 112.7 98.7) (end 112.7 98) (width 0.25) (layer B.Cu) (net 5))
 (via (at 113.6 100) (size 0.6) (drill 0.4) (layers F.Cu B.Cu) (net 5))
 (segment (start 100 113.6) (end 100.665 113.6) (width 0.25) (layer B.Cu) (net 6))
 (segment (start 100.665 113.6) (end 101.565 112.7) (width 0.25) (layer B.Cu) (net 6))
 (segment (start 101.565 112.7) (end 102 112.7) (width 0.25) (layer B.Cu) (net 6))
 (segment (start 100 113.6) (end 98.55 113.6) (width 0.25) (layer F.Cu) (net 6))
 (via (at 100 113.6) (size 0.6) (drill 0.4) (layers F.Cu B.Cu) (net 6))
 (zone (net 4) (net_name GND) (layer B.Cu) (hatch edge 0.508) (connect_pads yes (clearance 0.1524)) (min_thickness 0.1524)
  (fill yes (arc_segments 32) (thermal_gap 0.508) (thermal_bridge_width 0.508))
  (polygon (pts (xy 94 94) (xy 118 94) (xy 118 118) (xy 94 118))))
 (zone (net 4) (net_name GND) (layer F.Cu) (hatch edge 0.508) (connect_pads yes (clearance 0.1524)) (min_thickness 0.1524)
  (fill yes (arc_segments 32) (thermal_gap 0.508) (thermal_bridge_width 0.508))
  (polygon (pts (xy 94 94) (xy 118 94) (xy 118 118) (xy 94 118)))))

